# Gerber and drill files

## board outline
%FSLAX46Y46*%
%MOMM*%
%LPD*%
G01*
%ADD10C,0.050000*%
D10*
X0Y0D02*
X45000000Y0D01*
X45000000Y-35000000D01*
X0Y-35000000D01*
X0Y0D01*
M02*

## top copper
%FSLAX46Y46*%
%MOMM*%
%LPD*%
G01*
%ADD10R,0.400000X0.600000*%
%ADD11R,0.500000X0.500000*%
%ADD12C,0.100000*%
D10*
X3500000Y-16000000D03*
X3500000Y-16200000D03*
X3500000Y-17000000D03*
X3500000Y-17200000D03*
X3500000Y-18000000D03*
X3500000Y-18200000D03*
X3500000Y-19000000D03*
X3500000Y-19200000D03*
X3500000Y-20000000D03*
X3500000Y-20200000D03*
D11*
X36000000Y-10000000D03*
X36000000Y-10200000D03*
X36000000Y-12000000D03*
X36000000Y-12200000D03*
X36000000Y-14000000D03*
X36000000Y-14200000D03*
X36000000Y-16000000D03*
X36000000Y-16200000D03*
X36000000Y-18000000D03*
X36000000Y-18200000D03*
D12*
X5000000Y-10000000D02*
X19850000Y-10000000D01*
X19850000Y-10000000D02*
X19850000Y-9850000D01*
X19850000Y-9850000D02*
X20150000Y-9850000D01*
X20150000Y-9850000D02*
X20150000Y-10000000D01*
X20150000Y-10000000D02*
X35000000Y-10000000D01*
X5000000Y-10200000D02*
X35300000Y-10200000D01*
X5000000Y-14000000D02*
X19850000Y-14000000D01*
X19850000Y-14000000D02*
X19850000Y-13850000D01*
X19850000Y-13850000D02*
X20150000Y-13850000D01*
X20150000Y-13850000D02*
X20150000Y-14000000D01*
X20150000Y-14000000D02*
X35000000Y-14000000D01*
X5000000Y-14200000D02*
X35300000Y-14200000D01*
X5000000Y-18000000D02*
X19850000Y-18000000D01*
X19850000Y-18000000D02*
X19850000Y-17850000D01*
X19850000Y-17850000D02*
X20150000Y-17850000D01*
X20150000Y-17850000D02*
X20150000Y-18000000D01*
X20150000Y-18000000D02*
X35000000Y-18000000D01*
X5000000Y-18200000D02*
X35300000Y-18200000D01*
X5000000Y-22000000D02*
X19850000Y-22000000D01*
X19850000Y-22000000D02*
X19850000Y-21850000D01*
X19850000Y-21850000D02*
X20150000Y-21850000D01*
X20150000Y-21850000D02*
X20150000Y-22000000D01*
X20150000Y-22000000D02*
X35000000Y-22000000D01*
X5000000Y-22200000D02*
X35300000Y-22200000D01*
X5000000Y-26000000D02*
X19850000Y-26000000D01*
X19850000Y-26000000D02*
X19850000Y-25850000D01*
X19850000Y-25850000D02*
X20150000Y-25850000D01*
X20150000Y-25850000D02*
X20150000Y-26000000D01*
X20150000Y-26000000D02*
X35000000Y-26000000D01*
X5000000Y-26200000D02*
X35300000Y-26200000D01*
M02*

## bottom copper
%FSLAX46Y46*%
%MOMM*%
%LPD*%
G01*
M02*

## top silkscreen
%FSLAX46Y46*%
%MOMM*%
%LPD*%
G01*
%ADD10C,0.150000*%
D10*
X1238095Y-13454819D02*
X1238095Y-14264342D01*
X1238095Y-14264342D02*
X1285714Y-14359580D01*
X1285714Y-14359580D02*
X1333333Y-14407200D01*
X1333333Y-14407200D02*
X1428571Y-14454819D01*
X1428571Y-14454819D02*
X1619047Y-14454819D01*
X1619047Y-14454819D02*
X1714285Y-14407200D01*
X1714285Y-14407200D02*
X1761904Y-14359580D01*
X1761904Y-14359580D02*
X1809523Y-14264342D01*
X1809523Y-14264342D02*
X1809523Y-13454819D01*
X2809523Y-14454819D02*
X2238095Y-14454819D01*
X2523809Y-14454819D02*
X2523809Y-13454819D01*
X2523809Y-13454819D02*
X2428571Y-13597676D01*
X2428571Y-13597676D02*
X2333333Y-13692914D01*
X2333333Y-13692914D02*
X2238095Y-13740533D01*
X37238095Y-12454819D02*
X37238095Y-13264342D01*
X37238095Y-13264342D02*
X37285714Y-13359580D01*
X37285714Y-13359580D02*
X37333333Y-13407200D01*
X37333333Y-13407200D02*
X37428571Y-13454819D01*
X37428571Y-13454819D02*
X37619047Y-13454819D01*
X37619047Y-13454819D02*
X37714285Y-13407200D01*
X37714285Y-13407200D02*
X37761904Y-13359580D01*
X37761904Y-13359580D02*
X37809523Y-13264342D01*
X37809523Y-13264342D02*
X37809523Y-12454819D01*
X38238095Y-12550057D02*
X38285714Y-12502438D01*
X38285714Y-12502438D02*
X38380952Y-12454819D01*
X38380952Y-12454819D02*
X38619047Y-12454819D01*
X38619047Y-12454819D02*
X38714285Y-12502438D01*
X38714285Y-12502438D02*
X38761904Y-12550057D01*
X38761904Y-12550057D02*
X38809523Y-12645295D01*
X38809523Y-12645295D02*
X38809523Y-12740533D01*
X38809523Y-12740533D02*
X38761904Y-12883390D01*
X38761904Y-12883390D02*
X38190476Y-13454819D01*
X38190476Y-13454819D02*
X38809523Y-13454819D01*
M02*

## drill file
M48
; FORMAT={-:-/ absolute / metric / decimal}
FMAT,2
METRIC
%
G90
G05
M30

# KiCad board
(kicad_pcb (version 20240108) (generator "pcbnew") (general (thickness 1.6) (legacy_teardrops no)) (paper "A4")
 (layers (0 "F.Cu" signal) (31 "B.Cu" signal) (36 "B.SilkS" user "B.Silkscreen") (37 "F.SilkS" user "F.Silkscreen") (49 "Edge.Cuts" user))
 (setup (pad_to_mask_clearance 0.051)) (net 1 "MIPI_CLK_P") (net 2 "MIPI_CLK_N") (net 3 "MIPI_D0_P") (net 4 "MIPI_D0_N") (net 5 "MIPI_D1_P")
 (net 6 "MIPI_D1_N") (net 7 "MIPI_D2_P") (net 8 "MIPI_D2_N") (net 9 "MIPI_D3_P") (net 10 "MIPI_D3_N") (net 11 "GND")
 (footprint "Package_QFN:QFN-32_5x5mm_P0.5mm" (layer "F.Cu") (at 2 18)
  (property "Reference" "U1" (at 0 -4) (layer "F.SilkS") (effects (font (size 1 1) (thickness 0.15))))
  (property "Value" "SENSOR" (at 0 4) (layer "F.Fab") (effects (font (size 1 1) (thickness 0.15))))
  (pad "1" smd rect (at 1.5 -2) (size 0.4 0.6) (layers "F.Cu" "F.Paste" "F.Mask") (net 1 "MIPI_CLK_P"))
  (pad "2" smd rect (at 1.5 -1.8) (size 0.4 0.6) (layers "F.Cu" "F.Paste" "F.Mask") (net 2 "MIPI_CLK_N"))
  (pad "3" smd rect (at 1.5 -1) (size 0.4 0.6) (layers "F.Cu" "F.Paste" "F.Mask") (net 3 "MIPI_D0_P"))
  (pad "4" smd rect (at 1.5 -0.8) (size 0.4 0.6) (layers "F.Cu" "F.Paste" "F.Mask") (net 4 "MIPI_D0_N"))
  (pad "5" smd rect (at 1.5 0) (size 0.4 0.6) (layers "F.Cu" "F.Paste" "F.Mask") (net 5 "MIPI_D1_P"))
  (pad "6" smd rect (at 1.5 0.2) (size 0.4 0.6) (layers "F.Cu" "F.Paste" "F.Mask") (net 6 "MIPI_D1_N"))
  (pad "7" smd rect (at 1.5 1) (size 0.4 0.6) (layers "F.Cu" "F.Paste" "F.Mask") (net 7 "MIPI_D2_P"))
  (pad "8" smd rect (at 1.5 1.2) (size 0.4 0.6) (layers "F.Cu" "F.Paste" "F.Mask") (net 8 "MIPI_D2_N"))
  (pad "9" smd rect (at 1.5 2) (size 0.4 0.6) (layers "F.Cu" "F.Paste" "F.Mask") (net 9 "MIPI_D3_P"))
  (pad "10" smd rect (at 1.5 2.2) (size 0.4 0.6) (layers "F.Cu" "F.Paste" "F.Mask") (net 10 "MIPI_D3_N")))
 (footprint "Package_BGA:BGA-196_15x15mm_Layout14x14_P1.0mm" (layer "F.Cu") (at 38 18)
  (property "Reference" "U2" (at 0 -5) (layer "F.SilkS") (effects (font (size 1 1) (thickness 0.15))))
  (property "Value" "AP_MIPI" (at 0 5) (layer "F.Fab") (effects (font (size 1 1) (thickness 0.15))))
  (pad "A1" smd rect (at -2 -8) (size 0.5 0.5) (layers "F.Cu" "F.Paste" "F.Mask") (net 1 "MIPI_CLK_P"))
  (pad "A2" smd rect (at -2 -7.8) (size 0.5 0.5) (layers "F.Cu" "F.Paste" "F.Mask") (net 2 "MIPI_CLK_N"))
  (pad "B1" smd rect (at -2 -6) (size 0.5 0.5) (layers "F.Cu" "F.Paste" "F.Mask") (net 3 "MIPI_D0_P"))
  (pad "B2" smd rect (at -2 -5.8) (size 0.5 0.5) (layers "F.Cu" "F.Paste" "F.Mask") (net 4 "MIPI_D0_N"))
  (pad "C1" smd rect (at -2 -4) (size 0.5 0.5) (layers "F.Cu" "F.Paste" "F.Mask") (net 5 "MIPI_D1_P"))
  (pad "C2" smd rect (at -2 -3.8) (size 0.5 0.5) (layers "F.Cu" "F.Paste" "F.Mask") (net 6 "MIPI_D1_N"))
  (pad "D1" smd rect (at -2 -2) (size 0.5 0.5) (layers "F.Cu" "F.Paste" "F.Mask") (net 7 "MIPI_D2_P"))
  (pad "D2" smd rect (at -2 -1.8) (size 0.5 0.5) (layers "F.Cu" "F.Paste" "F.Mask") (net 8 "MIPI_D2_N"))
  (pad "E1" smd rect (at -2 0) (size 0.5 0.5) (layers "F.Cu" "F.Paste" "F.Mask") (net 9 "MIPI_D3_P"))
  (pad "E2" smd rect (at -2 0.2) (size 0.5 0.5) (layers "F.Cu" "F.Paste" "F.Mask") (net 10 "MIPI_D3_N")))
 (segment (start 5 10.0) (end 19.85 10.0) (width 0.1) (layer "F.Cu") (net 1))
 (segment (start 19.85 10.0) (end 19.85 9.850) (width 0.1) (layer "F.Cu") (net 1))
 (segment (start 19.85 9.850) (end 20.15 9.850) (width 0.1) (layer "F.Cu") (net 1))
 (segment (start 20.15 9.850) (end 20.15 10.0) (width 0.1) (layer "F.Cu") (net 1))
 (segment (start 20.15 10.0) (end 35 10.0) (width 0.1) (layer "F.Cu") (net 1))
 (segment (start 5 10.2) (end 35.3 10.2) (width 0.1) (layer "F.Cu") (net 2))
 (segment (start 5 14.0) (end 19.85 14.0) (width 0.1) (layer "F.Cu") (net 3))
 (segment (start 19.85 14.0) (end 19.85 13.850) (width 0.1) (layer "F.Cu") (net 3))
 (segment (start 19.85 13.850) (end 20.15 13.850) (width 0.1) (layer "F.Cu") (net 3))
 (segment (start 20.15 13.850) (end 20.15 14.0) (width 0.1) (layer "F.Cu") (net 3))
 (segment (start 20.15 14.0) (end 35 14.0) (width 0.1) (layer "F.Cu") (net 3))
 (segment (start 5 14.2) (end 35.3 14.2) (width 0.1) (layer "F.Cu") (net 4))
 (segment (start 5 18.0) (end 19.85 18.0) (width 0.1) (layer "F.Cu") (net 5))
 (segment (start 19.85 18.0) (end 19.85 17.850) (width 0.1) (layer "F.Cu") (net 5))
 (segment (start 19.85 17.850) (end 20.15 17.850) (width 0.1) (layer "F.Cu") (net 5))
 (segment (start 20.15 17.850) (end 20.15 18.0) (width 0.1) (layer "F.Cu") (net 5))
 (segment (start 20.15 18.0) (end 35 18.0) (width 0.1) (layer "F.Cu") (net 5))
 (segment (start 5 18.2) (end 35.3 18.2) (width 0.1) (layer "F.Cu") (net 6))
 (segment (start 5 22.0) (end 19.85 22.0) (width 0.1) (layer "F.Cu") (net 7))
 (segment (start 19.85 22.0) (end 19.85 21.850) (width 0.1) (layer "F.Cu") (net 7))
 (segment (start 19.85 21.850) (end 20.15 21.850) (width 0.1) (layer "F.Cu") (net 7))
 (segment (start 20.15 21.850) (end 20.15 22.0) (width 0.1) (layer "F.Cu") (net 7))
 (segment (start 20.15 22.0) (end 35 22.0) (width 0.1) (layer "F.Cu") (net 7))
 (segment (start 5 22.2) (end 35.3 22.2) (width 0.1) (layer "F.Cu") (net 8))
 (segment (start 5 26.0) (end 19.85 26.0) (width 0.1) (layer "F.Cu") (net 9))
 (segment (start 19.85 26.0) (end 19.85 25.850) (width 0.1) (layer "F.Cu") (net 9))
 (segment (start 19.85 25.850) (end 20.15 25.850) (width 0.1) (layer "F.Cu") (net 9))
 (segment (start 20.15 25.850) (end 20.15 26.0) (width 0.1) (layer "F.Cu") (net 9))
 (segment (start 20.15 26.0) (end 35 26.0) (width 0.1) (layer "F.Cu") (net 9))
 (segment (start 5 26.2) (end 35.3 26.2) (width 0.1) (layer "F.Cu") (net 10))
 (gr_rect (start 0 0) (end 45 35) (layer "Edge.Cuts") (width 0.05)))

